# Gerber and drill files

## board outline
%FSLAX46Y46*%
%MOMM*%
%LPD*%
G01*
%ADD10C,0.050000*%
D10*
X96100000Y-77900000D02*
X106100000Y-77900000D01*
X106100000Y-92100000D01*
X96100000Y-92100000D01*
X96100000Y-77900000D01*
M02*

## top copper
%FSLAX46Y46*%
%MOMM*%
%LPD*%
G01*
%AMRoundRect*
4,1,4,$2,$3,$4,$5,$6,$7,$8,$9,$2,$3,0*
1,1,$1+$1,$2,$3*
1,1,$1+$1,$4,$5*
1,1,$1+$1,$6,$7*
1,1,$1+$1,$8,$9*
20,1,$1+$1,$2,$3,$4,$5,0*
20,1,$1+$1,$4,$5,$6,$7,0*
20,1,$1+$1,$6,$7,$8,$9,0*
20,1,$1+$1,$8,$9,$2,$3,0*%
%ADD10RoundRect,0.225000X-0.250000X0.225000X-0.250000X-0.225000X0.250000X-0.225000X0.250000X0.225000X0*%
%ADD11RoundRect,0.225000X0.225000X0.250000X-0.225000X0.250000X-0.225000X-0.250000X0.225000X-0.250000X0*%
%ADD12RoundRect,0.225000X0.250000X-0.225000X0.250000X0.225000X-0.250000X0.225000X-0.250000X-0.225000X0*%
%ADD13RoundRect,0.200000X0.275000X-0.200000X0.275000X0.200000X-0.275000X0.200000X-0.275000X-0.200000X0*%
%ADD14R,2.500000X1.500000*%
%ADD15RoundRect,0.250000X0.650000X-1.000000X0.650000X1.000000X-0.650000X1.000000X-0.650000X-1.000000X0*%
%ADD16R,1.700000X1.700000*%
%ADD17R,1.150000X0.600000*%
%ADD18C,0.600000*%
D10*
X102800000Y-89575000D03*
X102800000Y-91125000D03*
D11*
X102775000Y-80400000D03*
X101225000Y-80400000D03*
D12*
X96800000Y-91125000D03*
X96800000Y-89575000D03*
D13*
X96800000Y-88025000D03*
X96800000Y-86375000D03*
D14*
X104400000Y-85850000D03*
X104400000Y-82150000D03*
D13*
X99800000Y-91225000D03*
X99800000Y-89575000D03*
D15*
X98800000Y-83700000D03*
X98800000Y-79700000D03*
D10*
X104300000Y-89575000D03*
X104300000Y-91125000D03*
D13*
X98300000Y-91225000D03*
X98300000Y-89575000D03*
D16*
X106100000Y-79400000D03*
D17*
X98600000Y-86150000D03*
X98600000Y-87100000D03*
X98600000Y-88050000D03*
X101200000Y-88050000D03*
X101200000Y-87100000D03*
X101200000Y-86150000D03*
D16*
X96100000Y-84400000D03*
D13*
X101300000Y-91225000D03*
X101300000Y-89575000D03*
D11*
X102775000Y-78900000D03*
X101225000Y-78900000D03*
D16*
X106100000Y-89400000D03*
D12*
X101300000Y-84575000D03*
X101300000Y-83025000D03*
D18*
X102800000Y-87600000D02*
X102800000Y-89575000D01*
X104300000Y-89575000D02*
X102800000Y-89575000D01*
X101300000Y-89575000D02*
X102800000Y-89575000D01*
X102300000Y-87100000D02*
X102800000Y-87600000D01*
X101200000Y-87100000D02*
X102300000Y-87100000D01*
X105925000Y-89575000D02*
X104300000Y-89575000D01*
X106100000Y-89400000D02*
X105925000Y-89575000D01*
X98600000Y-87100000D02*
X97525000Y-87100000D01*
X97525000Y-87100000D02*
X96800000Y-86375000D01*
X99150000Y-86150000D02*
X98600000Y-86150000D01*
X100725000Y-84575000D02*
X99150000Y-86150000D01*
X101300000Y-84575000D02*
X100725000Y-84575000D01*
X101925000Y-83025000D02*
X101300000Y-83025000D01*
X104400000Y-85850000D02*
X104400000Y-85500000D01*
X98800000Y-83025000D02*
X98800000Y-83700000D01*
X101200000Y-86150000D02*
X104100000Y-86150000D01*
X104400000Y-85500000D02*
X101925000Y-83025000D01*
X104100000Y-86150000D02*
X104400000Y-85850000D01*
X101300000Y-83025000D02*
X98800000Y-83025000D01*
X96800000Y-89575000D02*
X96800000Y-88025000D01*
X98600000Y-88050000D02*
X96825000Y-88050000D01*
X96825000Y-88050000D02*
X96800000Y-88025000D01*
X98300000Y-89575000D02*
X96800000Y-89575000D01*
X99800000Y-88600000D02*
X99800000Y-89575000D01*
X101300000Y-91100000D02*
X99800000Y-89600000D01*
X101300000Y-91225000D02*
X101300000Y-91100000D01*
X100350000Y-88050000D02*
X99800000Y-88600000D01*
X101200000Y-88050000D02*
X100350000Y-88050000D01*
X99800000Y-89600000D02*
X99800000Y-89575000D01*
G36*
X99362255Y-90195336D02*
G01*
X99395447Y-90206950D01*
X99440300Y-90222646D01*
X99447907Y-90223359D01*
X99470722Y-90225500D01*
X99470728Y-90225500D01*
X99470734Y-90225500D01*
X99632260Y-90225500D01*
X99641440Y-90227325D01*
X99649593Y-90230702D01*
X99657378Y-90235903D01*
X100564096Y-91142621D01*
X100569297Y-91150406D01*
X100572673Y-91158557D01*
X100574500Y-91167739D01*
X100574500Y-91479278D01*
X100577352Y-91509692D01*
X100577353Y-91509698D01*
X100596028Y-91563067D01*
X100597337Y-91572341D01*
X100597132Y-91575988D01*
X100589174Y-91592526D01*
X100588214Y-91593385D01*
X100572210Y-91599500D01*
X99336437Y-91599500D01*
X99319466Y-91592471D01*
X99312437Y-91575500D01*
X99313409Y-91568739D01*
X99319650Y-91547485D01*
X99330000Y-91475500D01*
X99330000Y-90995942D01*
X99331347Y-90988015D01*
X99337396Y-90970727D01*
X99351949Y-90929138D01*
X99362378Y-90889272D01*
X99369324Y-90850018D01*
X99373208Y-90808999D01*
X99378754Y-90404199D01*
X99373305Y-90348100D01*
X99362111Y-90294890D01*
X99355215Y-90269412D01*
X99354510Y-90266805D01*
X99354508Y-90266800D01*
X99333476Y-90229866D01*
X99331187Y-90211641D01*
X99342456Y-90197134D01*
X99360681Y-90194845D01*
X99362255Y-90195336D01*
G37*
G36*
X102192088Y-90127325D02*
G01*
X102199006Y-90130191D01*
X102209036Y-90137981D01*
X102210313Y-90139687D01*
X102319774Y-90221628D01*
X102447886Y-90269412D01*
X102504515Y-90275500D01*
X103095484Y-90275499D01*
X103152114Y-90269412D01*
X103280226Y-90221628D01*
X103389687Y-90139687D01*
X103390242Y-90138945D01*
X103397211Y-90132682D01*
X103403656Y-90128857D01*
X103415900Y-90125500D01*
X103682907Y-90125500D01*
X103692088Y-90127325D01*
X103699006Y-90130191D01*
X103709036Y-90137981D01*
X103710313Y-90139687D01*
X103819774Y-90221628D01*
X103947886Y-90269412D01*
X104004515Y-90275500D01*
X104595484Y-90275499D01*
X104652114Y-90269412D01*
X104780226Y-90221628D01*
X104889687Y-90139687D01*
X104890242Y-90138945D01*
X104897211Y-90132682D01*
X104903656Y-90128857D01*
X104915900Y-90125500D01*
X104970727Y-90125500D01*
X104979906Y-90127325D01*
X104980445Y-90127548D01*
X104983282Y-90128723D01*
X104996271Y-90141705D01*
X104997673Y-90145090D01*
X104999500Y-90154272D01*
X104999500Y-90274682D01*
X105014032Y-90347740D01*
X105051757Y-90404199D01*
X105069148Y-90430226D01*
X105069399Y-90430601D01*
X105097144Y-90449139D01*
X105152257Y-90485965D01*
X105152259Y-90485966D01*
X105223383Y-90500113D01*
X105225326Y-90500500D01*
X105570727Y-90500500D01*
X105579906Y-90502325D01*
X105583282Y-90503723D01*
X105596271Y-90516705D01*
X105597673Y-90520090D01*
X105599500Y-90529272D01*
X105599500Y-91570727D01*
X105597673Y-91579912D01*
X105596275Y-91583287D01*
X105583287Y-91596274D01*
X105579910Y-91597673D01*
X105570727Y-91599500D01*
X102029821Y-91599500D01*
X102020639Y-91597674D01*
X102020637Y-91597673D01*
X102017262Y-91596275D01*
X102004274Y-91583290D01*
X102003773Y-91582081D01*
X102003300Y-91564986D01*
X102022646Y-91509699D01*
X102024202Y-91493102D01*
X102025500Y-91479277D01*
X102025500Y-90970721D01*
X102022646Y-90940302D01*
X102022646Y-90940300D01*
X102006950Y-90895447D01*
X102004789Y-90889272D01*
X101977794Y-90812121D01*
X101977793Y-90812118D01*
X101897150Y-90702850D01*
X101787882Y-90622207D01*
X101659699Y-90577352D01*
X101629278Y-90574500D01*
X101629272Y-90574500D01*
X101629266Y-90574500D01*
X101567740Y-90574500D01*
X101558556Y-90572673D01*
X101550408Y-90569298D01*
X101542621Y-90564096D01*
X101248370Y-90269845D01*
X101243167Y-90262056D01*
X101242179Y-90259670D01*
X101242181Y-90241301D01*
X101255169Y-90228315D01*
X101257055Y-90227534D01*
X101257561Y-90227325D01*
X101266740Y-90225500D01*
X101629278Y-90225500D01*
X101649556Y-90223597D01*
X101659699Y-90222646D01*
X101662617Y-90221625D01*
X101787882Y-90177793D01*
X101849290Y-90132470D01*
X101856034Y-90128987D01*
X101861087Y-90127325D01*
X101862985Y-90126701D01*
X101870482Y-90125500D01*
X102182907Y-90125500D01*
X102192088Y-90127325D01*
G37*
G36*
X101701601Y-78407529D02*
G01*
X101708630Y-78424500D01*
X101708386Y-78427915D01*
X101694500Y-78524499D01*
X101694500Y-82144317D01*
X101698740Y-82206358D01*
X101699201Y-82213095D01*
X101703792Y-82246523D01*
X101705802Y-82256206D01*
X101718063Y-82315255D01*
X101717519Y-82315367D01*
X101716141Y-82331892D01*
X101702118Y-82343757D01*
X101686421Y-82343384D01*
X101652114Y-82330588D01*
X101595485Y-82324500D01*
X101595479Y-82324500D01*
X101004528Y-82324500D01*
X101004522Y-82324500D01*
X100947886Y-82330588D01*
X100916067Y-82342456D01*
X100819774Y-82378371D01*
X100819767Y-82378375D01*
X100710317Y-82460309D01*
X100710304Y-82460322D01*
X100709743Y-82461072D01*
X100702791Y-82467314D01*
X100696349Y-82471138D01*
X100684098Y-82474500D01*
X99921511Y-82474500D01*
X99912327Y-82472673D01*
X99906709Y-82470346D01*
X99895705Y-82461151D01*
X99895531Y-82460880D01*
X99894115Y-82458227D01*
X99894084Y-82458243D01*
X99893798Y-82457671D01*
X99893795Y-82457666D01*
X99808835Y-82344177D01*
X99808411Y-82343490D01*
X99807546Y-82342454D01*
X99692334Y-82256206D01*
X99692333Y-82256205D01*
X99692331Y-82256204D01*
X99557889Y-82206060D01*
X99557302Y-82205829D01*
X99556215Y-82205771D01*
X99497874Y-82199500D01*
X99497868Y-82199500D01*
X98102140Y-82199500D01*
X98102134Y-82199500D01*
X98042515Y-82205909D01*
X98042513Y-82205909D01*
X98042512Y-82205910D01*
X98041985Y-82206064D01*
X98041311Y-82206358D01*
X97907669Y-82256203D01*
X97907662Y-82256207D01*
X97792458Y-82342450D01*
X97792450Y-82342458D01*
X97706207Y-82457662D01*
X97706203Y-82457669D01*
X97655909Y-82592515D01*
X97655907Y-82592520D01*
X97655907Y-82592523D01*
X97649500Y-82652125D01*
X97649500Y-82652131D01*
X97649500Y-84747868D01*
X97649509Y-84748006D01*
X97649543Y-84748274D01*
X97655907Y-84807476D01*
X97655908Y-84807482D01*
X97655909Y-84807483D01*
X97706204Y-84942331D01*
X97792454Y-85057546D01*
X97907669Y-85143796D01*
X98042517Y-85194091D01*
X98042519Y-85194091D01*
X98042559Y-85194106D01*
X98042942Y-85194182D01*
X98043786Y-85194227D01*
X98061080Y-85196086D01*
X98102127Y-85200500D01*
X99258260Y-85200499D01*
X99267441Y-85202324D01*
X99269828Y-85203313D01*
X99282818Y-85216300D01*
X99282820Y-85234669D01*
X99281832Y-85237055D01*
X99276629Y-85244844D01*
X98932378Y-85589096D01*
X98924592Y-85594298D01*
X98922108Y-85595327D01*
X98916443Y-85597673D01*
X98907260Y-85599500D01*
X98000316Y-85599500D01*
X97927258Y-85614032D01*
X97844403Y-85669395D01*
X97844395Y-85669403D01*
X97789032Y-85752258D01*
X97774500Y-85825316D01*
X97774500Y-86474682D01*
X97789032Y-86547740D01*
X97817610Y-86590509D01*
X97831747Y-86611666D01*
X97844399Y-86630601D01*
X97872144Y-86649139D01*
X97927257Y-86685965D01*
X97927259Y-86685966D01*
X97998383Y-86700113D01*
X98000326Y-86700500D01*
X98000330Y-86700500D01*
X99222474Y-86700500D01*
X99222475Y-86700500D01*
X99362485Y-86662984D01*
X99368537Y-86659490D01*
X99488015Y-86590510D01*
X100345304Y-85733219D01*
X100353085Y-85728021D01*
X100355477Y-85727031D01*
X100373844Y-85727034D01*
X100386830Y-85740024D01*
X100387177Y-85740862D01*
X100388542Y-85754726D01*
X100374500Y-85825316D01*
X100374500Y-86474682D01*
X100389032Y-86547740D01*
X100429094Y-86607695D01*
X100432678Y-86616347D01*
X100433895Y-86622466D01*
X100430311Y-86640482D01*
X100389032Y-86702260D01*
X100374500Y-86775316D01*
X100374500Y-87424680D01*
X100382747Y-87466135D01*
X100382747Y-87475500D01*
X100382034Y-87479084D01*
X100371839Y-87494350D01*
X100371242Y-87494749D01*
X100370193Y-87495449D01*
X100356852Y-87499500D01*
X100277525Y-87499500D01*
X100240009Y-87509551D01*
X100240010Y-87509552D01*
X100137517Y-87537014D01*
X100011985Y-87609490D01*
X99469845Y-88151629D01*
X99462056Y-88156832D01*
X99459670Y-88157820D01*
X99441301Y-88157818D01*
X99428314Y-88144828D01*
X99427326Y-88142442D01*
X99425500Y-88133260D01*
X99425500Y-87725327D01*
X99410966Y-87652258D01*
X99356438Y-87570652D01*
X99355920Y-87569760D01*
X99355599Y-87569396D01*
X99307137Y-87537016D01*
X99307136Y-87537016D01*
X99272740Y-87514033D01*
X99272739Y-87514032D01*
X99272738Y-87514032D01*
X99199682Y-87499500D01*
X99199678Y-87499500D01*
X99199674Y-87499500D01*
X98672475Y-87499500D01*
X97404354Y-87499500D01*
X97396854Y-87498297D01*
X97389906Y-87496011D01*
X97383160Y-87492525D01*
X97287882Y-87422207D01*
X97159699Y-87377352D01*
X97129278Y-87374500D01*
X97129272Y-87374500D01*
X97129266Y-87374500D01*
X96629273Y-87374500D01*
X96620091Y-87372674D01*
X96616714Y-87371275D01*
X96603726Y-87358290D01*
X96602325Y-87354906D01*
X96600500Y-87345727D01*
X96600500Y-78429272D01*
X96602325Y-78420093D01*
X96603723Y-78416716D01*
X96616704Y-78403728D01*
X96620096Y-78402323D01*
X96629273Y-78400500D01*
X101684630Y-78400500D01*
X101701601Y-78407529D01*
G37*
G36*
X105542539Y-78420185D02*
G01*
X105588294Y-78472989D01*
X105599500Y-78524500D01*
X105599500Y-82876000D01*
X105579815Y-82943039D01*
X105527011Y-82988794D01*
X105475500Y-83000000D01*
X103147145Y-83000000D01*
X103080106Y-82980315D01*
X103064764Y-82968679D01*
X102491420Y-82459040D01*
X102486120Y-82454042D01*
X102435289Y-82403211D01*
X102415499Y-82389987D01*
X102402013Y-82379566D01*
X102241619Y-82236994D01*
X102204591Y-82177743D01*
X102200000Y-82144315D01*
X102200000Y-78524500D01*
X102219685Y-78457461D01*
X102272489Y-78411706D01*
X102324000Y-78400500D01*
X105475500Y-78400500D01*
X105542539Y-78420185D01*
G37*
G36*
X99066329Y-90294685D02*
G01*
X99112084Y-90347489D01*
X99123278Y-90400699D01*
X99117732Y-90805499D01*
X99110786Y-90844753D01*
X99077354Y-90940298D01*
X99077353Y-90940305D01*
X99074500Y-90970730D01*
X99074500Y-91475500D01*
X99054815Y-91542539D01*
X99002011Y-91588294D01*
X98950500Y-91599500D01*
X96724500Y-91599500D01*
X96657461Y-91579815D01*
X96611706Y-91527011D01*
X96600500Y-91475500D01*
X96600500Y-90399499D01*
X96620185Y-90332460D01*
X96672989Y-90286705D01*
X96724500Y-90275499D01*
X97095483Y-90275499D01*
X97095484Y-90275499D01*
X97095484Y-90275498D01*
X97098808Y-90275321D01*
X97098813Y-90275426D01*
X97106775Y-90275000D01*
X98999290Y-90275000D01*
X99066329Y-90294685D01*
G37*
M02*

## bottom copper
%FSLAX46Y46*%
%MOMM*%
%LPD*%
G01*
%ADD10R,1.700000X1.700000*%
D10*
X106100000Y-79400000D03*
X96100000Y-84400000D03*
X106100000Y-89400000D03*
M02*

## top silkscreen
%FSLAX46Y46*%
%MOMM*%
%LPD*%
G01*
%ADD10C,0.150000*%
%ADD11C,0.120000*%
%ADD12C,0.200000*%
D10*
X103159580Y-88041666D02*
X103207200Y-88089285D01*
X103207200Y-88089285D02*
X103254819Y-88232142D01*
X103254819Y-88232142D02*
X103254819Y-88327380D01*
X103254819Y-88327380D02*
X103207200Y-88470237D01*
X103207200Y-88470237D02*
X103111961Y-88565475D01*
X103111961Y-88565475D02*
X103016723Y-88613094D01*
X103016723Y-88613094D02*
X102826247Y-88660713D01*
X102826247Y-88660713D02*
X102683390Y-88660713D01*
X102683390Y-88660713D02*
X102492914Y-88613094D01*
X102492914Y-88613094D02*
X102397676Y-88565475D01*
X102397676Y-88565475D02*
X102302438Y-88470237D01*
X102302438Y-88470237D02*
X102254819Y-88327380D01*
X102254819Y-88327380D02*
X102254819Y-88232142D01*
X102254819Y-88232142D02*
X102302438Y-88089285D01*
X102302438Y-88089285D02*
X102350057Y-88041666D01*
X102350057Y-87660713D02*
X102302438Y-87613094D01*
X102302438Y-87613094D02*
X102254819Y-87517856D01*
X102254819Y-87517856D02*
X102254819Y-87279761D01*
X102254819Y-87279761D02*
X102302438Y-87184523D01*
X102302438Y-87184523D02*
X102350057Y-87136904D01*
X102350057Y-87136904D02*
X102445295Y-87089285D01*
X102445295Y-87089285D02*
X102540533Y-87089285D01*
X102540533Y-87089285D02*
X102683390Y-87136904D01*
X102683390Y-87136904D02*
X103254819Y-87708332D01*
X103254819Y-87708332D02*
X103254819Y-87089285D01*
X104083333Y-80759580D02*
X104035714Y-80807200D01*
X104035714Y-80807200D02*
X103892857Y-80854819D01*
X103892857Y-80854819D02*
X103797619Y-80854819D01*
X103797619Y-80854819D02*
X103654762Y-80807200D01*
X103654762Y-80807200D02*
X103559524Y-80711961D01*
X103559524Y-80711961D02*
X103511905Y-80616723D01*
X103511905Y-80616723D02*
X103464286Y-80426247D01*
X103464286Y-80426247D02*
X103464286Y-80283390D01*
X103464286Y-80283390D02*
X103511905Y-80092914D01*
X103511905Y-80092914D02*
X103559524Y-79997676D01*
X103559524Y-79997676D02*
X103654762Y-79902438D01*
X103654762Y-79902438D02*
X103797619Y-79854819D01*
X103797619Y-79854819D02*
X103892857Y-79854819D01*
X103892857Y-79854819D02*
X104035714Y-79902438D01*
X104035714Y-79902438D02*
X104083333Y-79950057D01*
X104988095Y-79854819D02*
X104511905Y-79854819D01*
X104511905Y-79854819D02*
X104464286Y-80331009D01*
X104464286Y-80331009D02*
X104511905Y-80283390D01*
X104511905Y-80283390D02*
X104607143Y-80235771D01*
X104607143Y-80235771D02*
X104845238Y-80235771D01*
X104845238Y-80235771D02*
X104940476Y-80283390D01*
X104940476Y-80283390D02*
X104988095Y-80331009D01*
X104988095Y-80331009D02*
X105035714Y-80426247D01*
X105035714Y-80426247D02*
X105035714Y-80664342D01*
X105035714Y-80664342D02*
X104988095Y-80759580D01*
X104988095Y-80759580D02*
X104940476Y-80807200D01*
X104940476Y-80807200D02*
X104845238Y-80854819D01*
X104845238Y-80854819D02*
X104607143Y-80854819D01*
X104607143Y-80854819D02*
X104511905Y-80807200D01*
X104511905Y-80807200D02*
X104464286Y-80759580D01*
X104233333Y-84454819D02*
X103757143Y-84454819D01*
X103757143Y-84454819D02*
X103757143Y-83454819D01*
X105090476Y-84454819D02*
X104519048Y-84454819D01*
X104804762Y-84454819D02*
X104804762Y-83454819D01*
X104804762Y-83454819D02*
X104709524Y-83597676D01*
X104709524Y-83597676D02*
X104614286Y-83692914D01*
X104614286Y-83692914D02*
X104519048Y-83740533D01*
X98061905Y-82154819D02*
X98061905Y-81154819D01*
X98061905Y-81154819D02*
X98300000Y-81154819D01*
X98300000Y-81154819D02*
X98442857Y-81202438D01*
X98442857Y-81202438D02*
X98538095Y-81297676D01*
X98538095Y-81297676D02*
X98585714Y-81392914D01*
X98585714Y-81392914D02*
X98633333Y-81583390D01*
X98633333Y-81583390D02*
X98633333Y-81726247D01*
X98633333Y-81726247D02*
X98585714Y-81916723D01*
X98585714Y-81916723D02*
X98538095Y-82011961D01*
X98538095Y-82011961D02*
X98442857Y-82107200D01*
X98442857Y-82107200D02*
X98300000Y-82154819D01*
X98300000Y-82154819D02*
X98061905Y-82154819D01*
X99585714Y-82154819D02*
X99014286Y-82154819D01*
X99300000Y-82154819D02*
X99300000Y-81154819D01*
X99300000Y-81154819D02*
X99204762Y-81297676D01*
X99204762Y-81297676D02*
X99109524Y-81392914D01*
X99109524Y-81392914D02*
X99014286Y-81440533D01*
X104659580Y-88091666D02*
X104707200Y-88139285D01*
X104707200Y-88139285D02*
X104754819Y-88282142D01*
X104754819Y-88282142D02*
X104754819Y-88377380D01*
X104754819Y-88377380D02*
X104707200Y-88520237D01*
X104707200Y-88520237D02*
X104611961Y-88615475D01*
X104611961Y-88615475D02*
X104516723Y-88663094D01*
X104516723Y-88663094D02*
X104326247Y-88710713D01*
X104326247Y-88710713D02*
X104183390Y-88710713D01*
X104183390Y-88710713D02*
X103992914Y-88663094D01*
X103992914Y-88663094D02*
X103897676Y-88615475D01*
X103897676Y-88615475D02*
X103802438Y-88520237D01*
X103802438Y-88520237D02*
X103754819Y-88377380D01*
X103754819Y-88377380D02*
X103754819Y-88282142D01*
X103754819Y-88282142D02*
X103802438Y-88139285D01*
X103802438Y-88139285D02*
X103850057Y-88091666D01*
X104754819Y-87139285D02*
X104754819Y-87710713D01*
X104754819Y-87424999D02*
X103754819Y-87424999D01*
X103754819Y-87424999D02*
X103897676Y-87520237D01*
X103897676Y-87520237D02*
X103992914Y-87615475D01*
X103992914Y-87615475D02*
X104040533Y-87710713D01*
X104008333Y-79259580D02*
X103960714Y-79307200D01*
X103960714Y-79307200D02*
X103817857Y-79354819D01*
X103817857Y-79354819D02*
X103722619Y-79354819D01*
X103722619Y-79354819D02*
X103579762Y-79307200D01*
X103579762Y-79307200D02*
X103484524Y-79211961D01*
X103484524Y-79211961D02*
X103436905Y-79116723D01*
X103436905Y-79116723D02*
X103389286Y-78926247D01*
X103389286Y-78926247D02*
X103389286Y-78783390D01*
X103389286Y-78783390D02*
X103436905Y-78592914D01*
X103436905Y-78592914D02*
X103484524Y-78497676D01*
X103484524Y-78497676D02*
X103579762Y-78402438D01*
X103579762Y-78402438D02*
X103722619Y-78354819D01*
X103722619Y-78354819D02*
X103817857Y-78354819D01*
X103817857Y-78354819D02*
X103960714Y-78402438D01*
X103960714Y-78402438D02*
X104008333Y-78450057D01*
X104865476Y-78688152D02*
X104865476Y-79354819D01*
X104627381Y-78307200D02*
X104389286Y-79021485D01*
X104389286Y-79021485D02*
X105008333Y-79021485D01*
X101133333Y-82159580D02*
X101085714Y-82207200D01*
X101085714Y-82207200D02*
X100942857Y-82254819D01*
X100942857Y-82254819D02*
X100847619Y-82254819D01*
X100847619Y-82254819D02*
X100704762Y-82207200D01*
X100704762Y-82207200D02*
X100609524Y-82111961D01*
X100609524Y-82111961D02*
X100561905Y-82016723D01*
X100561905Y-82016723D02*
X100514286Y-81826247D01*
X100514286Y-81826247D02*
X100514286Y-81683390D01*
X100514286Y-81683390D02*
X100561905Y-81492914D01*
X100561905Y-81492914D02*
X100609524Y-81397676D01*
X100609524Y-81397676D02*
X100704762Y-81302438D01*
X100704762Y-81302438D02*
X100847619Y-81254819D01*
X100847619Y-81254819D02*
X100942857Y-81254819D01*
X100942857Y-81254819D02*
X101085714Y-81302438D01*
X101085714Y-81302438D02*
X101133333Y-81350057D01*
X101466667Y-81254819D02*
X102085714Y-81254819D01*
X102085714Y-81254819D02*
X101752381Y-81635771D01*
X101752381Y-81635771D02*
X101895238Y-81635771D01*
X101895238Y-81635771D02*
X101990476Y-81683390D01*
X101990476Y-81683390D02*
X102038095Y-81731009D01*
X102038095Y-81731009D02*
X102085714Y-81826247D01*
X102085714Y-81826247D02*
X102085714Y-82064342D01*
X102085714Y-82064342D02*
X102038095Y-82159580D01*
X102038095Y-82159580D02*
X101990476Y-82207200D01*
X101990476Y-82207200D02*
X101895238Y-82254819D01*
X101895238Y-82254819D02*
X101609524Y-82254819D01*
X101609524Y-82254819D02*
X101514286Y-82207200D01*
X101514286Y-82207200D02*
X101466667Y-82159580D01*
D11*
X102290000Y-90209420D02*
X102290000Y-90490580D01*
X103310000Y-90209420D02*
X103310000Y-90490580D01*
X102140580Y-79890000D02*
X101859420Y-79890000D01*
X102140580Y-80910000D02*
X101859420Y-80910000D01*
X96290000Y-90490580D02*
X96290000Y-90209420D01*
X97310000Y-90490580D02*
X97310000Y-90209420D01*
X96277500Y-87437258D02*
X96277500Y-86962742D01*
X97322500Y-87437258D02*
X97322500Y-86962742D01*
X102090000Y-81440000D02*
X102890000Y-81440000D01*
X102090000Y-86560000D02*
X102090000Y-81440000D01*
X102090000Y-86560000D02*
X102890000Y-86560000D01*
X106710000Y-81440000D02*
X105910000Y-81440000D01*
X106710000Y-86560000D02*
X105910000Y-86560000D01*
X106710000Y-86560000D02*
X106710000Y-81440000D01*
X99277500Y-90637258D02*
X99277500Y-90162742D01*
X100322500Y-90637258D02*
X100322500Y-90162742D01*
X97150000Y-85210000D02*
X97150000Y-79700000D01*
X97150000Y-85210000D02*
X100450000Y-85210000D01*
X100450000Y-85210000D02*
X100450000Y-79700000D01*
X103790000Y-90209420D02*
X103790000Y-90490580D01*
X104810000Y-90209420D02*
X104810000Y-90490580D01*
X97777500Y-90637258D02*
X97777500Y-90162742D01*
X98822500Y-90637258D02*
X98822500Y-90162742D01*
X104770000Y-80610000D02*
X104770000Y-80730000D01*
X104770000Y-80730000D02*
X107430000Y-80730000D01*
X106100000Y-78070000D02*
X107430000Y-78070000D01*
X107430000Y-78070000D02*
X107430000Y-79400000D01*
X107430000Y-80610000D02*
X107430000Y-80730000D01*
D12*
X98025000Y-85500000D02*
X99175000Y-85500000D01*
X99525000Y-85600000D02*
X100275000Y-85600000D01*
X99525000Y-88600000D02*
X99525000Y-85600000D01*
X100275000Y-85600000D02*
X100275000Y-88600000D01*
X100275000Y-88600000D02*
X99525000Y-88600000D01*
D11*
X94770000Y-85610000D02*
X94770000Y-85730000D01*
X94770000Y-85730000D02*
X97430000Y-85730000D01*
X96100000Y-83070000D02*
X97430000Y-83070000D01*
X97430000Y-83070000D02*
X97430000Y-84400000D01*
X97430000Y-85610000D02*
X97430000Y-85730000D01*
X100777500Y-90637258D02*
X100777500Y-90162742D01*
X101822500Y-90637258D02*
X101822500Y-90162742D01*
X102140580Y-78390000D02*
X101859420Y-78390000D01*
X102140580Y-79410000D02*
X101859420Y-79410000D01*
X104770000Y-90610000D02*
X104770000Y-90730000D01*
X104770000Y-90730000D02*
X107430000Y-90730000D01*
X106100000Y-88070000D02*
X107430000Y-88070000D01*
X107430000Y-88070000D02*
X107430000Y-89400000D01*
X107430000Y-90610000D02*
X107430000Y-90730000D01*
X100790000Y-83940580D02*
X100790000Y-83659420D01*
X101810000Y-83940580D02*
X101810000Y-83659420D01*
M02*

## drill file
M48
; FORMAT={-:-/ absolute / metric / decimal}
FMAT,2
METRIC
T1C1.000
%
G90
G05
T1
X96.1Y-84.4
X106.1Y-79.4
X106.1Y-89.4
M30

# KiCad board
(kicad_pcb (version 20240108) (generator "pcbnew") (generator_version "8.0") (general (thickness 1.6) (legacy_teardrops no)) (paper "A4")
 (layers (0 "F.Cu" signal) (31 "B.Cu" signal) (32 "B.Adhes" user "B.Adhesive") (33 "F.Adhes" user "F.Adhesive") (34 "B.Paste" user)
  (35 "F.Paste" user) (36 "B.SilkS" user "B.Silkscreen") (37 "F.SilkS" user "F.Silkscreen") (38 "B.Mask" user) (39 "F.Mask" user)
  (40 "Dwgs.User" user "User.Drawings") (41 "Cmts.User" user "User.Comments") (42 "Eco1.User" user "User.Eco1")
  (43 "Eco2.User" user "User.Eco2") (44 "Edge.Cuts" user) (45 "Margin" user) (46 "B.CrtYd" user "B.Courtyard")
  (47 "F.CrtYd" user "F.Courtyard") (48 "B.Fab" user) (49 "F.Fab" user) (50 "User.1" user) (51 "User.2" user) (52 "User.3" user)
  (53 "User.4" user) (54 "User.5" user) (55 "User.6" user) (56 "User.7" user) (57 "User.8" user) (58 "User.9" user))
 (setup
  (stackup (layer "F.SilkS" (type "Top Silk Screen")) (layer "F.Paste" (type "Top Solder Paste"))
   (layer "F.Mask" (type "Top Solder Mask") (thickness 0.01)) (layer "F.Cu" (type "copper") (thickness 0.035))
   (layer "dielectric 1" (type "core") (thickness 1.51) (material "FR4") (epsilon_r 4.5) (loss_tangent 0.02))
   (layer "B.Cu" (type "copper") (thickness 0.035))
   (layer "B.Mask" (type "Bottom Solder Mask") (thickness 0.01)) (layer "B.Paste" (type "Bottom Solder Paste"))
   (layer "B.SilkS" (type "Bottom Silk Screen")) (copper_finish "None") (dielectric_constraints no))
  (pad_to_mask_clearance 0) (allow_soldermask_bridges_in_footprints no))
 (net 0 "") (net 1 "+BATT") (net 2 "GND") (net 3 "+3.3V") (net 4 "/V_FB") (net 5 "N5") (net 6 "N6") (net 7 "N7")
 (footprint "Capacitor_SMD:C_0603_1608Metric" (layer "F.Cu") (at 102.8 90.35 -90)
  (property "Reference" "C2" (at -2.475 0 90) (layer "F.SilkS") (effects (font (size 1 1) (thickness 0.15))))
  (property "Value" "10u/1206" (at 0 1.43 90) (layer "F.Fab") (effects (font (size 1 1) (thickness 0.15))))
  (fp_line (start -0.14058 0.51) (end 0.14058 0.51) (stroke (width 0.12) (type solid)) (layer "F.SilkS"))
  (fp_line (start -0.14058 -0.51) (end 0.14058 -0.51) (stroke (width 0.12) (type solid)) (layer "F.SilkS"))
  (pad "1" smd roundrect (at -0.775 0 270) (size 0.9 0.95) (layers "F.Cu" "F.Paste" "F.Mask") (roundrect_rratio 0.25) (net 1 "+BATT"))
  (pad "2" smd roundrect (at 0.775 0 270) (size 0.9 0.95) (layers "F.Cu" "F.Paste" "F.Mask") (roundrect_rratio 0.25) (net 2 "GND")))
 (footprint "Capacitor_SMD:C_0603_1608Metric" (layer "F.Cu") (at 102 80.4 180)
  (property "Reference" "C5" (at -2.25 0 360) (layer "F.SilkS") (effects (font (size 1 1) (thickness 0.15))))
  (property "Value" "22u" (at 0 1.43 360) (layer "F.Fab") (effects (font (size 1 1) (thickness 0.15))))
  (fp_line (start -0.14058 0.51) (end 0.14058 0.51) (stroke (width 0.12) (type solid)) (layer "F.SilkS"))
  (fp_line (start -0.14058 -0.51) (end 0.14058 -0.51) (stroke (width 0.12) (type solid)) (layer "F.SilkS"))
  (pad "1" smd roundrect (at -0.775 0 180) (size 0.9 0.95) (layers "F.Cu" "F.Paste" "F.Mask") (roundrect_rratio 0.25) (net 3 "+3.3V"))
  (pad "2" smd roundrect (at 0.775 0 180) (size 0.9 0.95) (layers "F.Cu" "F.Paste" "F.Mask") (roundrect_rratio 0.25) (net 2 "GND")))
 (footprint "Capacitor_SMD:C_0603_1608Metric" (layer "F.Cu") (at 96.8 90.35 90)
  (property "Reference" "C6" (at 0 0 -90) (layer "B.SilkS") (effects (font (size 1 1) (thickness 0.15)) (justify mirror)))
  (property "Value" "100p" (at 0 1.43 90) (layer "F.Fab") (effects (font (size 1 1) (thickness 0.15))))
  (fp_line (start -0.14058 -0.51) (end 0.14058 -0.51) (stroke (width 0.12) (type solid)) (layer "F.SilkS"))
  (fp_line (start -0.14058 0.51) (end 0.14058 0.51) (stroke (width 0.12) (type solid)) (layer "F.SilkS"))
  (pad "1" smd roundrect (at -0.775 0 90) (size 0.9 0.95) (layers "F.Cu" "F.Paste" "F.Mask") (roundrect_rratio 0.25) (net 3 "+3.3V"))
  (pad "2" smd roundrect (at 0.775 0 90) (size 0.9 0.95) (layers "F.Cu" "F.Paste" "F.Mask") (roundrect_rratio 0.25) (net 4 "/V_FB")))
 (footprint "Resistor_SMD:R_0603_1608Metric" (layer "F.Cu") (at 96.8 87.2 90)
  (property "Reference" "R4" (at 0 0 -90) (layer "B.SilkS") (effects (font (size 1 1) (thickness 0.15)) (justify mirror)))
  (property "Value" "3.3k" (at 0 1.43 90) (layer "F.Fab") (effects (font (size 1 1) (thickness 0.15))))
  (fp_line (start -0.237258 -0.5225) (end 0.237258 -0.5225) (stroke (width 0.12) (type solid)) (layer "F.SilkS"))
  (fp_line (start -0.237258 0.5225) (end 0.237258 0.5225) (stroke (width 0.12) (type solid)) (layer "F.SilkS"))
  (pad "1" smd roundrect (at -0.825 0 90) (size 0.8 0.95) (layers "F.Cu" "F.Paste" "F.Mask") (roundrect_rratio 0.25) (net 4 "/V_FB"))
  (pad "2" smd roundrect (at 0.825 0 90) (size 0.8 0.95) (layers "F.Cu" "F.Paste" "F.Mask") (roundrect_rratio 0.25) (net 2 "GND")))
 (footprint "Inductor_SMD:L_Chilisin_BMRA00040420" (layer "F.Cu") (at 104.4 84 90)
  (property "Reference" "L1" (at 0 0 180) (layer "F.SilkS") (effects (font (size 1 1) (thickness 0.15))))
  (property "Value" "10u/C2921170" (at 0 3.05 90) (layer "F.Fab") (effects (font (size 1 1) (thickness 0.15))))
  (fp_line (start 2.56 -2.31) (end 2.56 -1.51) (stroke (width 0.12) (type solid)) (layer "F.SilkS"))
  (fp_line (start -2.56 -2.31) (end 2.56 -2.31) (stroke (width 0.12) (type solid)) (layer "F.SilkS"))
  (fp_line (start -2.56 -2.31) (end -2.56 -1.51) (stroke (width 0.12) (type solid)) (layer "F.SilkS"))
  (fp_line (start 2.56 2.31) (end 2.56 1.51) (stroke (width 0.12) (type solid)) (layer "F.SilkS"))
  (fp_line (start -2.56 2.31) (end -2.56 1.51) (stroke (width 0.12) (type solid)) (layer "F.SilkS"))
  (fp_line (start -2.56 2.31) (end 2.56 2.31) (stroke (width 0.12) (type solid)) (layer "F.SilkS"))
  (pad "1" smd rect (at -1.85 0 90) (size 1.5 2.5) (layers "F.Cu" "F.Paste" "F.Mask") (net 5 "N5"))
  (pad "2" smd rect (at 1.85 0 90) (size 1.5 2.5) (layers "F.Cu" "F.Paste" "F.Mask") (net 3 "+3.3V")))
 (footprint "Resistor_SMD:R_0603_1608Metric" (layer "F.Cu") (at 99.8 90.4 90)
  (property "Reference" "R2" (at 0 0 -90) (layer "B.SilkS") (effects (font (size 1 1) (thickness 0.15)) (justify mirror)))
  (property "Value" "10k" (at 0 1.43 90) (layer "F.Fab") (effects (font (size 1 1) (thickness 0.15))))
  (fp_line (start -0.237258 -0.5225) (end 0.237258 -0.5225) (stroke (width 0.12) (type solid)) (layer "F.SilkS"))
  (fp_line (start -0.237258 0.5225) (end 0.237258 0.5225) (stroke (width 0.12) (type solid)) (layer "F.SilkS"))
  (pad "1" smd roundrect (at -0.825 0 90) (size 0.8 0.95) (layers "F.Cu" "F.Paste" "F.Mask") (roundrect_rratio 0.25) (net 2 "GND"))
  (pad "2" smd roundrect (at 0.825 0 90) (size 0.8 0.95) (layers "F.Cu" "F.Paste" "F.Mask") (roundrect_rratio 0.25) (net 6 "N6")))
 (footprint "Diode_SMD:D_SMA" (layer "F.Cu") (at 98.8 81.7 90)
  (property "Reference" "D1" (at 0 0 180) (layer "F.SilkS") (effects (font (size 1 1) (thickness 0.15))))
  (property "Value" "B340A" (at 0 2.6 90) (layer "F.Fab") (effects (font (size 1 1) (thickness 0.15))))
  (fp_line (start -3.51 -1.65) (end 2 -1.65) (stroke (width 0.12) (type solid)) (layer "F.SilkS"))
  (fp_line (start -3.51 -1.65) (end -3.51 1.65) (stroke (width 0.12) (type solid)) (layer "F.SilkS"))
  (fp_line (start -3.51 1.65) (end 2 1.65) (stroke (width 0.12) (type solid)) (layer "F.SilkS"))
  (pad "1" smd roundrect (at -2 0 90) (size 2.5 1.8) (layers "F.Cu" "F.Paste" "F.Mask") (roundrect_rratio 0.1388888889) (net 5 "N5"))
  (pad "2" smd roundrect (at 2 0 90) (size 2.5 1.8) (layers "F.Cu" "F.Paste" "F.Mask") (roundrect_rratio 0.1388888889) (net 2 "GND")))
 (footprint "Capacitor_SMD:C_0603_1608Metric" (layer "F.Cu") (at 104.3 90.35 -90)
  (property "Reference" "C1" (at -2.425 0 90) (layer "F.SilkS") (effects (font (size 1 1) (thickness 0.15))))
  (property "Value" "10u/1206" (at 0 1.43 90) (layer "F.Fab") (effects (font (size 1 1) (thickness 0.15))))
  (fp_line (start -0.14058 0.51) (end 0.14058 0.51) (stroke (width 0.12) (type solid)) (layer "F.SilkS"))
  (fp_line (start -0.14058 -0.51) (end 0.14058 -0.51) (stroke (width 0.12) (type solid)) (layer "F.SilkS"))
  (pad "1" smd roundrect (at -0.775 0 270) (size 0.9 0.95) (layers "F.Cu" "F.Paste" "F.Mask") (roundrect_rratio 0.25) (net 1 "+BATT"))
  (pad "2" smd roundrect (at 0.775 0 270) (size 0.9 0.95) (layers "F.Cu" "F.Paste" "F.Mask") (roundrect_rratio 0.25) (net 2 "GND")))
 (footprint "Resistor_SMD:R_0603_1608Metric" (layer "F.Cu") (at 98.3 90.4 90)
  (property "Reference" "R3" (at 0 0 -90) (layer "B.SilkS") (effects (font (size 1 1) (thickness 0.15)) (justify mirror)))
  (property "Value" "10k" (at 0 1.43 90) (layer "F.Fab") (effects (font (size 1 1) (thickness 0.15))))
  (fp_line (start -0.237258 -0.5225) (end 0.237258 -0.5225) (stroke (width 0.12) (type solid)) (layer "F.SilkS"))
  (fp_line (start -0.237258 0.5225) (end 0.237258 0.5225) (stroke (width 0.12) (type solid)) (layer "F.SilkS"))
  (pad "1" smd roundrect (at -0.825 0 90) (size 0.8 0.95) (layers "F.Cu" "F.Paste" "F.Mask") (roundrect_rratio 0.25) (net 3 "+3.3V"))
  (pad "2" smd roundrect (at 0.825 0 90) (size 0.8 0.95) (layers "F.Cu" "F.Paste" "F.Mask") (roundrect_rratio 0.25) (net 4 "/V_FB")))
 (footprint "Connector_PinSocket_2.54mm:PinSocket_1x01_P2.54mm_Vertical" (layer "F.Cu") (at 106.1 79.4)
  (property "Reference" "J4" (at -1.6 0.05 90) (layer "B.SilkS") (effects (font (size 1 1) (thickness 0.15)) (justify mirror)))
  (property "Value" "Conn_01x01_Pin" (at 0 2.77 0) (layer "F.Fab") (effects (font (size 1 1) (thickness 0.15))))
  (fp_line (start -1.33 1.21) (end -1.33 1.33) (stroke (width 0.12) (type solid)) (layer "F.SilkS"))
  (fp_line (start -1.33 1.33) (end 1.33 1.33) (stroke (width 0.12) (type solid)) (layer "F.SilkS"))
  (fp_line (start 0 -1.33) (end 1.33 -1.33) (stroke (width 0.12) (type solid)) (layer "F.SilkS"))
  (fp_line (start 1.33 -1.33) (end 1.33 0) (stroke (width 0.12) (type solid)) (layer "F.SilkS"))
  (fp_line (start 1.33 1.21) (end 1.33 1.33) (stroke (width 0.12) (type solid)) (layer "F.SilkS"))
  (pad "1" thru_hole rect (at 0 0) (size 1.7 1.7) (drill 1) (layers "*.Cu" "*.Mask") (remove_unused_layers no) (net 3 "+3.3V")))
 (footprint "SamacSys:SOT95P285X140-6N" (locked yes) (layer "F.Cu") (at 99.9 87.1)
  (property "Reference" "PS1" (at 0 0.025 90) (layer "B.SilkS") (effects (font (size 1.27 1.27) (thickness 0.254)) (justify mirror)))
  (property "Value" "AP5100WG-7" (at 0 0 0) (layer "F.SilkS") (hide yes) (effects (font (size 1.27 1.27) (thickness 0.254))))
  (fp_line (start -1.875 -1.6) (end -0.725 -1.6) (stroke (width 0.2) (type solid)) (layer "F.SilkS"))
  (fp_line (start -0.375 -1.5) (end 0.375 -1.5) (stroke (width 0.2) (type solid)) (layer "F.SilkS"))
  (fp_line (start -0.375 1.5) (end -0.375 -1.5) (stroke (width 0.2) (type solid)) (layer "F.SilkS"))
  (fp_line (start 0.375 -1.5) (end 0.375 1.5) (stroke (width 0.2) (type solid)) (layer "F.SilkS"))
  (fp_line (start 0.375 1.5) (end -0.375 1.5) (stroke (width 0.2) (type solid)) (layer "F.SilkS"))
  (pad "1" smd rect (at -1.3 -0.95 90) (size 0.6 1.15) (layers "F.Cu" "F.Paste" "F.Mask") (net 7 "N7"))
  (pad "2" smd rect (at -1.3 0 90) (size 0.6 1.15) (layers "F.Cu" "F.Paste" "F.Mask") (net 2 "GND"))
  (pad "3" smd rect (at -1.3 0.95 90) (size 0.6 1.15) (layers "F.Cu" "F.Paste" "F.Mask") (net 4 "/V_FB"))
  (pad "4" smd rect (at 1.3 0.95 90) (size 0.6 1.15) (layers "F.Cu" "F.Paste" "F.Mask") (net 6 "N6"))
  (pad "5" smd rect (at 1.3 0 90) (size 0.6 1.15) (layers "F.Cu" "F.Paste" "F.Mask") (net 1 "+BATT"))
  (pad "6" smd rect (at 1.3 -0.95 90) (size 0.6 1.15) (layers "F.Cu" "F.Paste" "F.Mask") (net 5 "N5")))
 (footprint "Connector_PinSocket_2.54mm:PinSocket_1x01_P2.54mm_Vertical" (layer "F.Cu") (at 96.1 84.4)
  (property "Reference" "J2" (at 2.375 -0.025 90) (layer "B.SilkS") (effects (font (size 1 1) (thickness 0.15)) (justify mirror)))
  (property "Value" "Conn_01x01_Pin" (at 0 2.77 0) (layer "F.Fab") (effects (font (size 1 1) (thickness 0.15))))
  (fp_line (start -1.33 1.21) (end -1.33 1.33) (stroke (width 0.12) (type solid)) (layer "F.SilkS"))
  (fp_line (start -1.33 1.33) (end 1.33 1.33) (stroke (width 0.12) (type solid)) (layer "F.SilkS"))
  (fp_line (start 0 -1.33) (end 1.33 -1.33) (stroke (width 0.12) (type solid)) (layer "F.SilkS"))
  (fp_line (start 1.33 -1.33) (end 1.33 0) (stroke (width 0.12) (type solid)) (layer "F.SilkS"))
  (fp_line (start 1.33 1.21) (end 1.33 1.33) (stroke (width 0.12) (type solid)) (layer "F.SilkS"))
  (pad "1" thru_hole rect (at 0 0) (size 1.7 1.7) (drill 1) (layers "*.Cu" "*.Mask") (remove_unused_layers no) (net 2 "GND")))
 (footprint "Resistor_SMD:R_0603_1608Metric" (layer "F.Cu") (at 101.3 90.4 90)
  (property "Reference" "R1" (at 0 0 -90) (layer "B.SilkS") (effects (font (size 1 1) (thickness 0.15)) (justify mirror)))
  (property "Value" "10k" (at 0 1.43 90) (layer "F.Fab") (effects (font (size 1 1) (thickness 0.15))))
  (fp_line (start -0.237258 -0.5225) (end 0.237258 -0.5225) (stroke (width 0.12) (type solid)) (layer "F.SilkS"))
  (fp_line (start -0.237258 0.5225) (end 0.237258 0.5225) (stroke (width 0.12) (type solid)) (layer "F.SilkS"))
  (pad "1" smd roundrect (at -0.825 0 90) (size 0.8 0.95) (layers "F.Cu" "F.Paste" "F.Mask") (roundrect_rratio 0.25) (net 6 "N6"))
  (pad "2" smd roundrect (at 0.825 0 90) (size 0.8 0.95) (layers "F.Cu" "F.Paste" "F.Mask") (roundrect_rratio 0.25) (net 1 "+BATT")))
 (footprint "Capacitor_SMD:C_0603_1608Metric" (layer "F.Cu") (at 102 78.9 180)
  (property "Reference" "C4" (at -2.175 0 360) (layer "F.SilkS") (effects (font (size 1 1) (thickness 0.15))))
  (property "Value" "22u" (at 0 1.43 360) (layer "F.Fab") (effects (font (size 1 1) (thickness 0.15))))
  (fp_line (start -0.14058 0.51) (end 0.14058 0.51) (stroke (width 0.12) (type solid)) (layer "F.SilkS"))
  (fp_line (start -0.14058 -0.51) (end 0.14058 -0.51) (stroke (width 0.12) (type solid)) (layer "F.SilkS"))
  (pad "1" smd roundrect (at -0.775 0 180) (size 0.9 0.95) (layers "F.Cu" "F.Paste" "F.Mask") (roundrect_rratio 0.25) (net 3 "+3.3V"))
  (pad "2" smd roundrect (at 0.775 0 180) (size 0.9 0.95) (layers "F.Cu" "F.Paste" "F.Mask") (roundrect_rratio 0.25) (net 2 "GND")))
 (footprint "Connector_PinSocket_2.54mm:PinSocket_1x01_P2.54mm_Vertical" (layer "F.Cu") (at 106.1 89.4)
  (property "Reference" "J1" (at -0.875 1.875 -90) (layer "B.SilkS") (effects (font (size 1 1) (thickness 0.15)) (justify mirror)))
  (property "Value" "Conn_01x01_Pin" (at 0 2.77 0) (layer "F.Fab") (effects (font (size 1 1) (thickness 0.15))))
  (fp_line (start -1.33 1.21) (end -1.33 1.33) (stroke (width 0.12) (type solid)) (layer "F.SilkS"))
  (fp_line (start -1.33 1.33) (end 1.33 1.33) (stroke (width 0.12) (type solid)) (layer "F.SilkS"))
  (fp_line (start 0 -1.33) (end 1.33 -1.33) (stroke (width 0.12) (type solid)) (layer "F.SilkS"))
  (fp_line (start 1.33 -1.33) (end 1.33 0) (stroke (width 0.12) (type solid)) (layer "F.SilkS"))
  (fp_line (start 1.33 1.21) (end 1.33 1.33) (stroke (width 0.12) (type solid)) (layer "F.SilkS"))
  (pad "1" thru_hole rect (at 0 0) (size 1.7 1.7) (drill 1) (layers "*.Cu" "*.Mask") (remove_unused_layers no) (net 1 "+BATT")))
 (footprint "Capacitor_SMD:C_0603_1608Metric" (layer "F.Cu") (at 101.3 83.8 90)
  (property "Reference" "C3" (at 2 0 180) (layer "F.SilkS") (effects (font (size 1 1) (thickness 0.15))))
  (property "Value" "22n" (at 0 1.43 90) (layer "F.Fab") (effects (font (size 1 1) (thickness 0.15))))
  (fp_line (start -0.14058 -0.51) (end 0.14058 -0.51) (stroke (width 0.12) (type solid)) (layer "F.SilkS"))
  (fp_line (start -0.14058 0.51) (end 0.14058 0.51) (stroke (width 0.12) (type solid)) (layer "F.SilkS"))
  (pad "1" smd roundrect (at -0.775 0 90) (size 0.9 0.95) (layers "F.Cu" "F.Paste" "F.Mask") (roundrect_rratio 0.25) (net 7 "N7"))
  (pad "2" smd roundrect (at 0.775 0 90) (size 0.9 0.95) (layers "F.Cu" "F.Paste" "F.Mask") (roundrect_rratio 0.25) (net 5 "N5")))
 (gr_rect (start 96.1 77.9) (end 106.1 92.1) (stroke (width 0.05) (type default)) (fill none) (layer "Edge.Cuts"))
 (segment (start 102.8 87.6) (end 102.8 89.575) (width 0.6) (layer "F.Cu") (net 1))
 (segment (start 104.3 89.575) (end 102.8 89.575) (width 0.6) (layer "F.Cu") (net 1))
 (segment (start 101.3 89.575) (end 102.8 89.575) (width 0.6) (layer "F.Cu") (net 1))
 (segment (start 102.3 87.1) (end 102.8 87.6) (width 0.6) (layer "F.Cu") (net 1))
 (segment (start 101.2 87.1) (end 102.3 87.1) (width 0.6) (layer "F.Cu") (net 1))
 (segment (start 105.925 89.575) (end 104.3 89.575) (width 0.6) (layer "F.Cu") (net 1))
 (segment (start 106.1 89.4) (end 105.925 89.575) (width 0.6) (layer "F.Cu") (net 1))
 (segment (start 98.6 87.1) (end 97.525 87.1) (width 0.6) (layer "F.Cu") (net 2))
 (segment (start 97.525 87.1) (end 96.8 86.375) (width 0.6) (layer "F.Cu") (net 2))
 (segment (start 99.15 86.15) (end 98.6 86.15) (width 0.6) (layer "F.Cu") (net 7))
 (segment (start 100.725 84.575) (end 99.15 86.15) (width 0.6) (layer "F.Cu") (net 7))
 (segment (start 101.3 84.575) (end 100.725 84.575) (width 0.6) (layer "F.Cu") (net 7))
 (segment (start 101.925 83.025) (end 101.3 83.025) (width 0.6) (layer "F.Cu") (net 5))
 (segment (start 104.4 85.85) (end 104.4 85.5) (width 0.6) (layer "F.Cu") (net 5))
 (segment (start 98.8 83.025) (end 98.8 83.7) (width 0.6) (layer "F.Cu") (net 5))
 (segment (start 101.2 86.15) (end 104.1 86.15) (width 0.6) (layer "F.Cu") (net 5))
 (segment (start 104.4 85.5) (end 101.925 83.025) (width 0.6) (layer "F.Cu") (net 5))
 (segment (start 104.1 86.15) (end 104.4 85.85) (width 0.6) (layer "F.Cu") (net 5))
 (segment (start 101.3 83.025) (end 98.8 83.025) (width 0.6) (layer "F.Cu") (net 5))
 (segment (start 96.8 89.575) (end 96.8 88.025) (width 0.6) (layer "F.Cu") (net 4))
 (segment (start 98.6 88.05) (end 96.825 88.05) (width 0.6) (layer "F.Cu") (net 4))
 (segment (start 96.825 88.05) (end 96.8 88.025) (width 0.6) (layer "F.Cu") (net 4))
 (segment (start 98.3 89.575) (end 96.8 89.575) (width 0.6) (layer "F.Cu") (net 4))
 (segment (start 99.8 88.6) (end 99.8 89.575) (width 0.6) (layer "F.Cu") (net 6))
 (segment (start 101.3 91.1) (end 99.8 89.6) (width 0.6) (layer "F.Cu") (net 6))
 (segment (start 101.3 91.225) (end 101.3 91.1) (width 0.6) (layer "F.Cu") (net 6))
 (segment (start 100.35 88.05) (end 99.8 88.6) (width 0.6) (layer "F.Cu") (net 6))
 (segment (start 101.2 88.05) (end 100.35 88.05) (width 0.6) (layer "F.Cu") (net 6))
 (segment (start 99.8 89.6) (end 99.8 89.575) (width 0.6) (layer "F.Cu") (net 6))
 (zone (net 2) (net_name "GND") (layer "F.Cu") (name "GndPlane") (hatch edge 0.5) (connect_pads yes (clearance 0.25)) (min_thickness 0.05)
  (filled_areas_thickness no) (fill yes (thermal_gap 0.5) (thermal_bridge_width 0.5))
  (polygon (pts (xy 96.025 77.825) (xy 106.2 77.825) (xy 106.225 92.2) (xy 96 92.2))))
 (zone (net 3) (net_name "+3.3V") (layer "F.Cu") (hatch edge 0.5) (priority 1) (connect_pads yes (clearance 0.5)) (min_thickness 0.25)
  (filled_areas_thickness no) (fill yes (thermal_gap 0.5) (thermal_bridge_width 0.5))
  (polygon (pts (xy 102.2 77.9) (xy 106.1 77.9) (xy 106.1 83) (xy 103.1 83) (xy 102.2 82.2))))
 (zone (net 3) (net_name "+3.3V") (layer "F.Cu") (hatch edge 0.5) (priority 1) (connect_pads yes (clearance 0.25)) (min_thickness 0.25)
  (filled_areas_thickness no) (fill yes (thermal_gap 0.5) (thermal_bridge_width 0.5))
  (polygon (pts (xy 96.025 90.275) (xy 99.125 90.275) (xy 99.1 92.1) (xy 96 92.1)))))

